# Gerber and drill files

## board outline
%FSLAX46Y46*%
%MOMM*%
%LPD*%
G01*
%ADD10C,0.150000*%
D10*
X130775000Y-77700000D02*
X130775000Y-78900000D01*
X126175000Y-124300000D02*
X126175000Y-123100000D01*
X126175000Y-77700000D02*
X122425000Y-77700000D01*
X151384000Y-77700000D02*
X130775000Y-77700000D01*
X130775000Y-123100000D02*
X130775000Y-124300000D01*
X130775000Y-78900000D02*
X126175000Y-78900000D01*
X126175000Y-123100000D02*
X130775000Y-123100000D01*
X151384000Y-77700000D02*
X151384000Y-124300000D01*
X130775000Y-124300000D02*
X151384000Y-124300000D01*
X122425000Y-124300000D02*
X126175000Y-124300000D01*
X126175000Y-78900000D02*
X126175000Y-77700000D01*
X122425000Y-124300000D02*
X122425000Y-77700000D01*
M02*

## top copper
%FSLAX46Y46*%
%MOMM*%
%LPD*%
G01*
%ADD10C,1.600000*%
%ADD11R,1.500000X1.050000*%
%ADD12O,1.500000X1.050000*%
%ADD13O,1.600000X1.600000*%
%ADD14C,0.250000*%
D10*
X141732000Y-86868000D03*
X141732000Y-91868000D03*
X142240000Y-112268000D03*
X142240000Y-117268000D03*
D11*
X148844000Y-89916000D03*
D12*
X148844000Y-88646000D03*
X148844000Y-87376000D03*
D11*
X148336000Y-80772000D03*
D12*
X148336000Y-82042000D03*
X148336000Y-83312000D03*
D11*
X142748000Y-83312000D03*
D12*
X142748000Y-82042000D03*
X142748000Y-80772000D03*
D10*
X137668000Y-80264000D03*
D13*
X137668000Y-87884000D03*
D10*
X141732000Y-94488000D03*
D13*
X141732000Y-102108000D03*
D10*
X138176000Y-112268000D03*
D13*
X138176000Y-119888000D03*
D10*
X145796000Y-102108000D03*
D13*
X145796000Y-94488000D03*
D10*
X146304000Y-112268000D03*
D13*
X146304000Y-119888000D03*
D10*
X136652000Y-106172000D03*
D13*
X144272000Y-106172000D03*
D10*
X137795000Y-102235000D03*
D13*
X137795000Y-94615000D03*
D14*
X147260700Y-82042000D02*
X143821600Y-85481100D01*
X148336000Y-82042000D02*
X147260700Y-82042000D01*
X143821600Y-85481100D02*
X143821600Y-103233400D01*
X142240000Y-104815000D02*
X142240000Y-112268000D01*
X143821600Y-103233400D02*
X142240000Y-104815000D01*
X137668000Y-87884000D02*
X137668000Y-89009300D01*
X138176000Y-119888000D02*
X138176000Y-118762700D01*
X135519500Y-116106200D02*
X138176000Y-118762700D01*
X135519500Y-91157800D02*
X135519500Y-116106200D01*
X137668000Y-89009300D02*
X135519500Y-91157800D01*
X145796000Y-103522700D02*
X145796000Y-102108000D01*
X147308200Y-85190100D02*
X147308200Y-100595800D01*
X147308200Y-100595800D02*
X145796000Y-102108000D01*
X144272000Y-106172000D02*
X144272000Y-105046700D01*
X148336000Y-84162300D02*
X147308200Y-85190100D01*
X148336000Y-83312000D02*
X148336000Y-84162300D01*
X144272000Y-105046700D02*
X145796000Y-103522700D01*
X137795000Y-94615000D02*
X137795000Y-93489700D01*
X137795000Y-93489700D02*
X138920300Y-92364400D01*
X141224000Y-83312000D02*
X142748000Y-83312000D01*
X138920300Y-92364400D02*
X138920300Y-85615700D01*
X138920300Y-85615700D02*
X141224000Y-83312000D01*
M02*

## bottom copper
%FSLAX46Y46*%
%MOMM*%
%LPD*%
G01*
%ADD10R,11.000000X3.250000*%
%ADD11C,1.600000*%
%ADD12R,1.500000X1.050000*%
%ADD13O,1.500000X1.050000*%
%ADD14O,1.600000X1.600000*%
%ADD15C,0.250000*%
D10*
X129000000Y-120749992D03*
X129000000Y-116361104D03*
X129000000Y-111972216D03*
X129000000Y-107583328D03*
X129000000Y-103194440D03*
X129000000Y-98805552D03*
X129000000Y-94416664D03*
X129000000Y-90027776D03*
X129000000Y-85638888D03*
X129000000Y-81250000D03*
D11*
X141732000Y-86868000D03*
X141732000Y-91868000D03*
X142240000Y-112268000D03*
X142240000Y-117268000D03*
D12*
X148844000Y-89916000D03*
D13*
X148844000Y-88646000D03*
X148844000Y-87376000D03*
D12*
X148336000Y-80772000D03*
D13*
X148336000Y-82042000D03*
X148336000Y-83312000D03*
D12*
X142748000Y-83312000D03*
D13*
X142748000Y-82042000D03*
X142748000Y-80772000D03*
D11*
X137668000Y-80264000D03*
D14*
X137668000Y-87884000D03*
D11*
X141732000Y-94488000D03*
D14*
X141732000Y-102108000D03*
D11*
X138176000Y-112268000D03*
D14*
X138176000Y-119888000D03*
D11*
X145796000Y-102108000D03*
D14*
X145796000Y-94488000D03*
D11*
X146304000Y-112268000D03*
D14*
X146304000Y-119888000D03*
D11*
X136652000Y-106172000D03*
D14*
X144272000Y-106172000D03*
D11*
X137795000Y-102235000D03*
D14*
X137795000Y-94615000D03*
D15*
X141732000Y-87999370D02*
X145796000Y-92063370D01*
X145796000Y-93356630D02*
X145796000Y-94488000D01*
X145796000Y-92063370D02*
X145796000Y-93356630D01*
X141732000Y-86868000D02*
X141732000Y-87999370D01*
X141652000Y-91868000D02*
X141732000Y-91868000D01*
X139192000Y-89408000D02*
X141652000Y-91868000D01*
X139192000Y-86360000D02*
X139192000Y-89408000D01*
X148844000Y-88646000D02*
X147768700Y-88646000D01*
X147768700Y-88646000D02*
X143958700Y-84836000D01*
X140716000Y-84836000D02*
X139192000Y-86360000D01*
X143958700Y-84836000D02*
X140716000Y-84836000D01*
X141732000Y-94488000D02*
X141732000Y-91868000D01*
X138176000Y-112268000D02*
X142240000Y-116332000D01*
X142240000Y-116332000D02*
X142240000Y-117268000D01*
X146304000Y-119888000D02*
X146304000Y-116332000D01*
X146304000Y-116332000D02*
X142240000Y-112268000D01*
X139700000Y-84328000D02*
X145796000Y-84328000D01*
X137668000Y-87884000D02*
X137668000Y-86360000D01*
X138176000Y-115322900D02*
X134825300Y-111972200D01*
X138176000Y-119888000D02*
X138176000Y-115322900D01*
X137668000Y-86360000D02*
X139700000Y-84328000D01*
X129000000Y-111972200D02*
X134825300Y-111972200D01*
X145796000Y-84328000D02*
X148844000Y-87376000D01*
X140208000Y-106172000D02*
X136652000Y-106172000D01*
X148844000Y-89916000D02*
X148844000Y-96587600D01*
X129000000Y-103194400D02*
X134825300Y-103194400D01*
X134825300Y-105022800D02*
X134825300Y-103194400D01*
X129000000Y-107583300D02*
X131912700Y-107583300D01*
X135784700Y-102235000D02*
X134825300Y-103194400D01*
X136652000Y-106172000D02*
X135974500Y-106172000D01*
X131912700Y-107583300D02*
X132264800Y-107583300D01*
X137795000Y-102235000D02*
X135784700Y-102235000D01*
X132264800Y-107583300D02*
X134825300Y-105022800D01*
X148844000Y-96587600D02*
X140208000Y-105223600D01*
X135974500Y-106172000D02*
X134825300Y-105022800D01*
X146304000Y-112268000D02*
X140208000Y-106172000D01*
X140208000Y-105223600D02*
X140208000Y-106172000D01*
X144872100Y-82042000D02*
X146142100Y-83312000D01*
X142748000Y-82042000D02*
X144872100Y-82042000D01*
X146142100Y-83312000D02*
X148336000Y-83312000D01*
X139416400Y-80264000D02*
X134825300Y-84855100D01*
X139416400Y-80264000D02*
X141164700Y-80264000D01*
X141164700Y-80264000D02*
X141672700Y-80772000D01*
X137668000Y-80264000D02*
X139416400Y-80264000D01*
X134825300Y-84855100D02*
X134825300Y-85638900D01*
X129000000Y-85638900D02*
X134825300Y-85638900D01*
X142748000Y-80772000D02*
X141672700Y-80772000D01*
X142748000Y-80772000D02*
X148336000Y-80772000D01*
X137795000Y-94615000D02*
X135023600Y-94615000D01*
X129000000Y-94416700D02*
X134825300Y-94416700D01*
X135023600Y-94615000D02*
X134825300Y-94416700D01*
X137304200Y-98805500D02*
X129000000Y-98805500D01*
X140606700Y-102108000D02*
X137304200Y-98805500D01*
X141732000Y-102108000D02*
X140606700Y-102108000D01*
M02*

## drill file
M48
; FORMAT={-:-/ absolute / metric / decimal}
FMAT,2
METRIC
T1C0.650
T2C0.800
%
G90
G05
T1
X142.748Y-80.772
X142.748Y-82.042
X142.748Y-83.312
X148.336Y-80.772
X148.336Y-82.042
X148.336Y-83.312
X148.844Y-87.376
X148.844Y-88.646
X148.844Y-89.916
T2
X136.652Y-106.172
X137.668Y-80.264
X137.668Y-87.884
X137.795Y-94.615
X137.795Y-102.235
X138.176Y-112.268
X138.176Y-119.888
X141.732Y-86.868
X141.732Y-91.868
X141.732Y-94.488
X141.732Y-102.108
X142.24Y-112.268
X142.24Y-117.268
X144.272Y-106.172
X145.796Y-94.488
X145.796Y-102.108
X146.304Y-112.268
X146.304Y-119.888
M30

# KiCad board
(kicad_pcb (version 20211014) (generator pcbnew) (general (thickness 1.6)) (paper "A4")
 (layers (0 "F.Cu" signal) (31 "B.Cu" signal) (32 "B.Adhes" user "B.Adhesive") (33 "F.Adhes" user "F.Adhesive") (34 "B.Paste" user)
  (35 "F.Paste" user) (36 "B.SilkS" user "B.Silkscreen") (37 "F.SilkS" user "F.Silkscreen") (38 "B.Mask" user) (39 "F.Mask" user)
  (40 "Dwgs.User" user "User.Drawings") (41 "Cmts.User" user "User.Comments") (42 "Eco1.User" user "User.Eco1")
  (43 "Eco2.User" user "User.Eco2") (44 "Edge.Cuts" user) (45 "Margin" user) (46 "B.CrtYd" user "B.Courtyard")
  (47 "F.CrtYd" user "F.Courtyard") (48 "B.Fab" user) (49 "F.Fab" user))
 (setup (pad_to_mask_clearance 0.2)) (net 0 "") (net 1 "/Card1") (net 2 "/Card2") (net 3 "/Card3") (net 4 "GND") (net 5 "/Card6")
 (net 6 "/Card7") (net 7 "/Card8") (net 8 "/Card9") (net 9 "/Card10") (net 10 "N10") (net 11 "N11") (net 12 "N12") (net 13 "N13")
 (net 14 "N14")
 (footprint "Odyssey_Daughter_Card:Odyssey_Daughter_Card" (layer "F.Cu") (at 129 101)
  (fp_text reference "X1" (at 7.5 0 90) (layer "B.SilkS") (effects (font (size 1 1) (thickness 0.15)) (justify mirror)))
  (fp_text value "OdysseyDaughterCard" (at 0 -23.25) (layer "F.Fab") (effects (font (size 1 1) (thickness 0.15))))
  (pad "1" smd rect locked (at 0 19.749992) (size 11 3.25) (layers "B.Cu" "B.Mask") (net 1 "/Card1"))
  (pad "2" smd rect locked (at 0 15.361104) (size 11 3.25) (layers "B.Cu" "B.Mask") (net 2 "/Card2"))
  (pad "3" smd rect locked (at 0 10.972216) (size 11 3.25) (layers "B.Cu" "B.Mask") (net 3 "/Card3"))
  (pad "4" smd rect locked (at 0 6.583328) (size 11 3.25) (layers "B.Cu" "B.Mask") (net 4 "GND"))
  (pad "5" smd rect locked (at 0 2.19444) (size 11 3.25) (layers "B.Cu" "B.Mask") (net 4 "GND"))
  (pad "6" smd rect locked (at 0 -2.194448) (size 11 3.25) (layers "B.Cu" "B.Mask") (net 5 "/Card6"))
  (pad "7" smd rect locked (at 0 -6.583336) (size 11 3.25) (layers "B.Cu" "B.Mask") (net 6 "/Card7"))
  (pad "8" smd rect locked (at 0 -10.972224) (size 11 3.25) (layers "B.Cu" "B.Mask") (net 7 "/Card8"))
  (pad "9" smd rect locked (at 0 -15.361112) (size 11 3.25) (layers "B.Cu" "B.Mask") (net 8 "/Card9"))
  (pad "10" smd rect locked (at 0 -19.75) (size 11 3.25) (layers "B.Cu" "B.Mask") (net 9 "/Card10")))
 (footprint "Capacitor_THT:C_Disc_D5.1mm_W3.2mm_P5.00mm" (layer "F.Cu") (at 141.732 86.868 -90)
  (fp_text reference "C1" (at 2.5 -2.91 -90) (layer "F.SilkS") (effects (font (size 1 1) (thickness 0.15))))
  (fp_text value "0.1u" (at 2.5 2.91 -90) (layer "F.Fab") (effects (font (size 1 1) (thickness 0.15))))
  (pad "1" thru_hole circle locked (at 0 0 270) (size 1.6 1.6) (drill 0.8) (layers *.Cu *.Mask) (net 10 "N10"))
  (pad "2" thru_hole circle locked (at 5 0 270) (size 1.6 1.6) (drill 0.8) (layers *.Cu *.Mask) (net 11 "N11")))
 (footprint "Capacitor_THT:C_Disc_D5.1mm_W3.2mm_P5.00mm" (layer "F.Cu") (at 142.24 112.268 -90)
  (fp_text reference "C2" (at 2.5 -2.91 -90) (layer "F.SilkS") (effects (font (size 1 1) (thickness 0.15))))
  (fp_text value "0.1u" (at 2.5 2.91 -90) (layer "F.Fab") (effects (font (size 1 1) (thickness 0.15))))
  (pad "1" thru_hole circle locked (at 0 0 270) (size 1.6 1.6) (drill 0.8) (layers *.Cu *.Mask) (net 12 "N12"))
  (pad "2" thru_hole circle locked (at 5 0 270) (size 1.6 1.6) (drill 0.8) (layers *.Cu *.Mask) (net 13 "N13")))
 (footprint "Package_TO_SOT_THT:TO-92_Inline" (layer "F.Cu") (at 148.844 89.916 90)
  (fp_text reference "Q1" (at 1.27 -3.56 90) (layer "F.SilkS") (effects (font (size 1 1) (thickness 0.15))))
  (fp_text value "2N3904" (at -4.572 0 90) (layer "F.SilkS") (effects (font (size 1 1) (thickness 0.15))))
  (pad "1" thru_hole rect locked (at 0 0 90) (size 1.05 1.5) (drill 0.65) (layers *.Cu *.Mask) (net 4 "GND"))
  (pad "2" thru_hole oval locked (at 1.27 0 90) (size 1.05 1.5) (drill 0.65) (layers *.Cu *.Mask) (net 11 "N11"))
  (pad "3" thru_hole oval locked (at 2.54 0 90) (size 1.05 1.5) (drill 0.65) (layers *.Cu *.Mask) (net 3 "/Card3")))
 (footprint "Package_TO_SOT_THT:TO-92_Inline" (layer "F.Cu") (at 148.336 80.772 -90)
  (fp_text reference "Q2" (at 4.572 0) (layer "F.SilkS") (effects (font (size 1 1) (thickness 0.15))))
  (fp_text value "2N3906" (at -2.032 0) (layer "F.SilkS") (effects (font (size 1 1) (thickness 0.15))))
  (pad "1" thru_hole rect locked (at 0 0 270) (size 1.05 1.5) (drill 0.65) (layers *.Cu *.Mask) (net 8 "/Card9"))
  (pad "2" thru_hole oval locked (at 1.27 0 270) (size 1.05 1.5) (drill 0.65) (layers *.Cu *.Mask) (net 12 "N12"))
  (pad "3" thru_hole oval locked (at 2.54 0 270) (size 1.05 1.5) (drill 0.65) (layers *.Cu *.Mask) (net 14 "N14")))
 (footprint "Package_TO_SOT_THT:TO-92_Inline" (layer "F.Cu") (at 142.748 83.312 90)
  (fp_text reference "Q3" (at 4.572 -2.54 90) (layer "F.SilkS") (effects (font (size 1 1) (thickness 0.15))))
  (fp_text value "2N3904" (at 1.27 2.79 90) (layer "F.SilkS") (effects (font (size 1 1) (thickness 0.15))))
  (pad "1" thru_hole rect locked (at 0 0 90) (size 1.05 1.5) (drill 0.65) (layers *.Cu *.Mask) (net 6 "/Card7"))
  (pad "2" thru_hole oval locked (at 1.27 0 90) (size 1.05 1.5) (drill 0.65) (layers *.Cu *.Mask) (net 14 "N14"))
  (pad "3" thru_hole oval locked (at 2.54 0 90) (size 1.05 1.5) (drill 0.65) (layers *.Cu *.Mask) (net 8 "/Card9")))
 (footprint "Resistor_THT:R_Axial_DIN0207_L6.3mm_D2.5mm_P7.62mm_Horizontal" (layer "F.Cu") (at 137.668 80.264 -90)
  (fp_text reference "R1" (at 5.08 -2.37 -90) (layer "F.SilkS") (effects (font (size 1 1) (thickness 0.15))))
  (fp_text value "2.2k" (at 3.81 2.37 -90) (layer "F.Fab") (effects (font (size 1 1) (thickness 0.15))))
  (pad "1" thru_hole circle locked (at 0 0 270) (size 1.6 1.6) (drill 0.8) (layers *.Cu *.Mask) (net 8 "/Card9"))
  (pad "2" thru_hole oval locked (at 7.62 0 270) (size 1.6 1.6) (drill 0.8) (layers *.Cu *.Mask) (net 3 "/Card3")))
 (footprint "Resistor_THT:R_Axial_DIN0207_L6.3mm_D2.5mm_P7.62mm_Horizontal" (layer "F.Cu") (at 141.732 94.488 -90)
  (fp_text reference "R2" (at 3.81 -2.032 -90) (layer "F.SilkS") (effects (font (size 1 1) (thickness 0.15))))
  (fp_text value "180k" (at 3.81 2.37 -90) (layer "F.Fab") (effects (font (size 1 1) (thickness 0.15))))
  (pad "1" thru_hole circle locked (at 0 0 270) (size 1.6 1.6) (drill 0.8) (layers *.Cu *.Mask) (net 11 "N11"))
  (pad "2" thru_hole oval locked (at 7.62 0 270) (size 1.6 1.6) (drill 0.8) (layers *.Cu *.Mask) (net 5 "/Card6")))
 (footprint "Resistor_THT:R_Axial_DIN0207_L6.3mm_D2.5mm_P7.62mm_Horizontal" (layer "F.Cu") (at 138.176 112.268 -90)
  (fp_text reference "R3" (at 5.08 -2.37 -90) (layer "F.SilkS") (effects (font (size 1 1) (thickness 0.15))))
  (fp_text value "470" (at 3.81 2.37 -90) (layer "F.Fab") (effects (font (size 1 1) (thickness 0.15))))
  (pad "1" thru_hole circle locked (at 0 0 270) (size 1.6 1.6) (drill 0.8) (layers *.Cu *.Mask) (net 13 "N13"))
  (pad "2" thru_hole oval locked (at 7.62 0 270) (size 1.6 1.6) (drill 0.8) (layers *.Cu *.Mask) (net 3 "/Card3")))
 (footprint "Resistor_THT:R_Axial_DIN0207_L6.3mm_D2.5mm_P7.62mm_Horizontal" (layer "F.Cu") (at 145.796 102.108 90)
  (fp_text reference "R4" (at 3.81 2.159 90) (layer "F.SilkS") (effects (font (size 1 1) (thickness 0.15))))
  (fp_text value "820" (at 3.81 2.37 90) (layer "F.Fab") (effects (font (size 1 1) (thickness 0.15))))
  (pad "1" thru_hole circle locked (at 0 0 90) (size 1.6 1.6) (drill 0.8) (layers *.Cu *.Mask) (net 14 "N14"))
  (pad "2" thru_hole oval locked (at 7.62 0 90) (size 1.6 1.6) (drill 0.8) (layers *.Cu *.Mask) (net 10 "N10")))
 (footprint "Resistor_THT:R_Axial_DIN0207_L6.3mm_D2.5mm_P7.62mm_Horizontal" (layer "F.Cu") (at 146.304 112.268 -90)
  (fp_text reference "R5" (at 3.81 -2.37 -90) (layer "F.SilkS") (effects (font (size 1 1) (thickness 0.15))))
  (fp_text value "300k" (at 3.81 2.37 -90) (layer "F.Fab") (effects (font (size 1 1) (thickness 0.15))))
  (pad "1" thru_hole circle locked (at 0 0 270) (size 1.6 1.6) (drill 0.8) (layers *.Cu *.Mask) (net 4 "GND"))
  (pad "2" thru_hole oval locked (at 7.62 0 270) (size 1.6 1.6) (drill 0.8) (layers *.Cu *.Mask) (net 12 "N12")))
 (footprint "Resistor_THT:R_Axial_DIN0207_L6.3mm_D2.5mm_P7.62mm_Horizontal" (layer "F.Cu") (at 136.652 106.172)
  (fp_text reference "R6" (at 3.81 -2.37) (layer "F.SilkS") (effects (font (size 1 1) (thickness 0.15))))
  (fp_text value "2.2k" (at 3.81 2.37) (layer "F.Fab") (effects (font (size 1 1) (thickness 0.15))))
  (pad "1" thru_hole circle locked (at 0 0) (size 1.6 1.6) (drill 0.8) (layers *.Cu *.Mask) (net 4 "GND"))
  (pad "2" thru_hole oval locked (at 7.62 0) (size 1.6 1.6) (drill 0.8) (layers *.Cu *.Mask) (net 14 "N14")))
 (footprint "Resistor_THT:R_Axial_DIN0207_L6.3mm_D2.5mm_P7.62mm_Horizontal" (layer "F.Cu") (at 137.795 102.235 90)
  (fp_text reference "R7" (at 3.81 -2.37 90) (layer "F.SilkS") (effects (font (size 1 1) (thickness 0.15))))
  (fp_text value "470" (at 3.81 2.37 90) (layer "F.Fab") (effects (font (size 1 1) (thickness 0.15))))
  (pad "1" thru_hole circle locked (at 0 0 90) (size 1.6 1.6) (drill 0.8) (layers *.Cu *.Mask) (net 4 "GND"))
  (pad "2" thru_hole oval locked (at 7.62 0 90) (size 1.6 1.6) (drill 0.8) (layers *.Cu *.Mask) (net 6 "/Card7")))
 (gr_line (start 130.775 77.7) (end 130.775 78.9) (layer "Edge.Cuts") (width 0.15))
 (gr_line (start 126.175 124.3) (end 126.175 123.1) (layer "Edge.Cuts") (width 0.15))
 (gr_line (start 126.175 77.7) (end 122.425 77.7) (layer "Edge.Cuts") (width 0.15))
 (gr_line (start 151.384 77.7) (end 130.775 77.7) (layer "Edge.Cuts") (width 0.15))
 (gr_line (start 130.775 123.1) (end 130.775 124.3) (layer "Edge.Cuts") (width 0.15))
 (gr_line (start 130.775 78.9) (end 126.175 78.9) (layer "Edge.Cuts") (width 0.15))
 (gr_line (start 126.175 123.1) (end 130.775 123.1) (layer "Edge.Cuts") (width 0.15))
 (gr_line (start 151.384 77.7) (end 151.384 124.3) (layer "Edge.Cuts") (width 0.15))
 (gr_line (start 130.775 124.3) (end 151.384 124.3) (layer "Edge.Cuts") (width 0.15))
 (gr_line (start 122.425 124.3) (end 126.175 124.3) (layer "Edge.Cuts") (width 0.15))
 (gr_line (start 126.175 78.9) (end 126.175 77.7) (layer "Edge.Cuts") (width 0.15))
 (gr_line (start 122.425 124.3) (end 122.425 77.7) (layer "Edge.Cuts") (width 0.15))
 (segment (start 141.732 87.99937) (end 145.796 92.06337) (width 0.25) (layer "B.Cu") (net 10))
 (segment (start 145.796 93.35663) (end 145.796 94.488) (width 0.25) (layer "B.Cu") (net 10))
 (segment (start 145.796 92.06337) (end 145.796 93.35663) (width 0.25) (layer "B.Cu") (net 10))
 (segment (start 141.732 86.868) (end 141.732 87.99937) (width 0.25) (layer "B.Cu") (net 10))
 (segment (start 141.652 91.868) (end 141.732 91.868) (width 0.25) (layer "B.Cu") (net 11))
 (segment (start 139.192 89.408) (end 141.652 91.868) (width 0.25) (layer "B.Cu") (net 11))
 (segment (start 139.192 86.36) (end 139.192 89.408) (width 0.25) (layer "B.Cu") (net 11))
 (segment (start 148.844 88.646) (end 147.7687 88.646) (width 0.25) (layer "B.Cu") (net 11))
 (segment (start 147.7687 88.646) (end 143.9587 84.836) (width 0.25) (layer "B.Cu") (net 11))
 (segment (start 140.716 84.836) (end 139.192 86.36) (width 0.25) (layer "B.Cu") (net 11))
 (segment (start 143.9587 84.836) (end 140.716 84.836) (width 0.25) (layer "B.Cu") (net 11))
 (segment (start 141.732 94.488) (end 141.732 91.868) (width 0.25) (layer "B.Cu") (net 11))
 (segment (start 138.176 112.268) (end 142.24 116.332) (width 0.25) (layer "B.Cu") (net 13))
 (segment (start 142.24 116.332) (end 142.24 117.268) (width 0.25) (layer "B.Cu") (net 13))
 (segment (start 147.2607 82.042) (end 143.8216 85.4811) (width 0.25) (layer "F.Cu") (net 12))
 (segment (start 148.336 82.042) (end 147.2607 82.042) (width 0.25) (layer "F.Cu") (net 12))
 (segment (start 143.8216 85.4811) (end 143.8216 103.2334) (width 0.25) (layer "F.Cu") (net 12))
 (segment (start 142.24 104.815) (end 142.24 112.268) (width 0.25) (layer "F.Cu") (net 12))
 (segment (start 143.8216 103.2334) (end 142.24 104.815) (width 0.25) (layer "F.Cu") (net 12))
 (segment (start 146.304 119.888) (end 146.304 116.332) (width 0.25) (layer "B.Cu") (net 12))
 (segment (start 146.304 116.332) (end 142.24 112.268) (width 0.25) (layer "B.Cu") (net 12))
 (segment (start 137.668 87.884) (end 137.668 89.0093) (width 0.25) (layer "F.Cu") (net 3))
 (segment (start 138.176 119.888) (end 138.176 118.7627) (width 0.25) (layer "F.Cu") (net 3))
 (segment (start 135.5195 116.1062) (end 138.176 118.7627) (width 0.25) (layer "F.Cu") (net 3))
 (segment (start 135.5195 91.1578) (end 135.5195 116.1062) (width 0.25) (layer "F.Cu") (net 3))
 (segment (start 137.668 89.0093) (end 135.5195 91.1578) (width 0.25) (layer "F.Cu") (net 3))
 (segment (start 139.7 84.328) (end 145.796 84.328) (width 0.25) (layer "B.Cu") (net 3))
 (segment (start 137.668 87.884) (end 137.668 86.36) (width 0.25) (layer "B.Cu") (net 3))
 (segment (start 138.176 115.3229) (end 134.8253 111.9722) (width 0.25) (layer "B.Cu") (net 3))
 (segment (start 138.176 119.888) (end 138.176 115.3229) (width 0.25) (layer "B.Cu") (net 3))
 (segment (start 137.668 86.36) (end 139.7 84.328) (width 0.25) (layer "B.Cu") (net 3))
 (segment (start 129 111.9722) (end 134.8253 111.9722) (width 0.25) (layer "B.Cu") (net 3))
 (segment (start 145.796 84.328) (end 148.844 87.376) (width 0.25) (layer "B.Cu") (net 3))
 (segment (start 140.208 106.172) (end 136.652 106.172) (width 0.25) (layer "B.Cu") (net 4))
 (segment (start 148.844 89.916) (end 148.844 96.5876) (width 0.25) (layer "B.Cu") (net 4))
 (segment (start 129 103.1944) (end 134.8253 103.1944) (width 0.25) (layer "B.Cu") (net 4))
 (segment (start 134.8253 105.0228) (end 134.8253 103.1944) (width 0.25) (layer "B.Cu") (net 4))
 (segment (start 129 107.5833) (end 131.9127 107.5833) (width 0.25) (layer "B.Cu") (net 4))
 (segment (start 135.7847 102.235) (end 134.8253 103.1944) (width 0.25) (layer "B.Cu") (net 4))
 (segment (start 136.652 106.172) (end 135.9745 106.172) (width 0.25) (layer "B.Cu") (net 4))
 (segment (start 131.9127 107.5833) (end 132.2648 107.5833) (width 0.25) (layer "B.Cu") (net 4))
 (segment (start 137.795 102.235) (end 135.7847 102.235) (width 0.25) (layer "B.Cu") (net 4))
 (segment (start 132.2648 107.5833) (end 134.8253 105.0228) (width 0.25) (layer "B.Cu") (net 4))
 (segment (start 148.844 96.5876) (end 140.208 105.2236) (width 0.25) (layer "B.Cu") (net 4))
 (segment (start 135.9745 106.172) (end 134.8253 105.0228) (width 0.25) (layer "B.Cu") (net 4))
 (segment (start 146.304 112.268) (end 140.208 106.172) (width 0.25) (layer "B.Cu") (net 4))
 (segment (start 140.208 105.2236) (end 140.208 106.172) (width 0.25) (layer "B.Cu") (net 4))
 (segment (start 145.796 103.5227) (end 145.796 102.108) (width 0.25) (layer "F.Cu") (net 14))
 (segment (start 147.3082 85.1901) (end 147.3082 100.5958) (width 0.25) (layer "F.Cu") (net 14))
 (segment (start 147.3082 100.5958) (end 145.796 102.108) (width 0.25) (layer "F.Cu") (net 14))
 (segment (start 144.272 106.172) (end 144.272 105.0467) (width 0.25) (layer "F.Cu") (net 14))
 (segment (start 148.336 84.1623) (end 147.3082 85.1901) (width 0.25) (layer "F.Cu") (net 14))
 (segment (start 148.336 83.312) (end 148.336 84.1623) (width 0.25) (layer "F.Cu") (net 14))
 (segment (start 144.272 105.0467) (end 145.796 103.5227) (width 0.25) (layer "F.Cu") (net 14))
 (segment (start 144.8721 82.042) (end 146.1421 83.312) (width 0.25) (layer "B.Cu") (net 14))
 (segment (start 142.748 82.042) (end 144.8721 82.042) (width 0.25) (layer "B.Cu") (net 14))
 (segment (start 146.1421 83.312) (end 148.336 83.312) (width 0.25) (layer "B.Cu") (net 14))
 (segment (start 139.4164 80.264) (end 134.8253 84.8551) (width 0.25) (layer "B.Cu") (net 8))
 (segment (start 139.4164 80.264) (end 141.1647 80.264) (width 0.25) (layer "B.Cu") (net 8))
 (segment (start 141.1647 80.264) (end 141.6727 80.772) (width 0.25) (layer "B.Cu") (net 8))
 (segment (start 137.668 80.264) (end 139.4164 80.264) (width 0.25) (layer "B.Cu") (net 8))
 (segment (start 134.8253 84.8551) (end 134.8253 85.6389) (width 0.25) (layer "B.Cu") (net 8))
 (segment (start 129 85.6389) (end 134.8253 85.6389) (width 0.25) (layer "B.Cu") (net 8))
 (segment (start 142.748 80.772) (end 141.6727 80.772) (width 0.25) (layer "B.Cu") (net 8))
 (segment (start 142.748 80.772) (end 148.336 80.772) (width 0.25) (layer "B.Cu") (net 8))
 (segment (start 137.795 94.615) (end 137.795 93.4897) (width 0.25) (layer "F.Cu") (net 6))
 (segment (start 137.795 93.4897) (end 138.9203 92.3644) (width 0.25) (layer "F.Cu") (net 6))
 (segment (start 141.224 83.312) (end 142.748 83.312) (width 0.25) (layer "F.Cu") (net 6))
 (segment (start 138.9203 92.3644) (end 138.9203 85.6157) (width 0.25) (layer "F.Cu") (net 6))
 (segment (start 138.9203 85.6157) (end 141.224 83.312) (width 0.25) (layer "F.Cu") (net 6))
 (segment (start 137.795 94.615) (end 135.0236 94.615) (width 0.25) (layer "B.Cu") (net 6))
 (segment (start 129 94.4167) (end 134.8253 94.4167) (width 0.25) (layer "B.Cu") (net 6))
 (segment (start 135.0236 94.615) (end 134.8253 94.4167) (width 0.25) (layer "B.Cu") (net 6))
 (segment (start 137.3042 98.8055) (end 129 98.8055) (width 0.25) (layer "B.Cu") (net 5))
 (segment (start 140.6067 102.108) (end 137.3042 98.8055) (width 0.25) (layer "B.Cu") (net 5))
 (segment (start 141.732 102.108) (end 140.6067 102.108) (width 0.25) (layer "B.Cu") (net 5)))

